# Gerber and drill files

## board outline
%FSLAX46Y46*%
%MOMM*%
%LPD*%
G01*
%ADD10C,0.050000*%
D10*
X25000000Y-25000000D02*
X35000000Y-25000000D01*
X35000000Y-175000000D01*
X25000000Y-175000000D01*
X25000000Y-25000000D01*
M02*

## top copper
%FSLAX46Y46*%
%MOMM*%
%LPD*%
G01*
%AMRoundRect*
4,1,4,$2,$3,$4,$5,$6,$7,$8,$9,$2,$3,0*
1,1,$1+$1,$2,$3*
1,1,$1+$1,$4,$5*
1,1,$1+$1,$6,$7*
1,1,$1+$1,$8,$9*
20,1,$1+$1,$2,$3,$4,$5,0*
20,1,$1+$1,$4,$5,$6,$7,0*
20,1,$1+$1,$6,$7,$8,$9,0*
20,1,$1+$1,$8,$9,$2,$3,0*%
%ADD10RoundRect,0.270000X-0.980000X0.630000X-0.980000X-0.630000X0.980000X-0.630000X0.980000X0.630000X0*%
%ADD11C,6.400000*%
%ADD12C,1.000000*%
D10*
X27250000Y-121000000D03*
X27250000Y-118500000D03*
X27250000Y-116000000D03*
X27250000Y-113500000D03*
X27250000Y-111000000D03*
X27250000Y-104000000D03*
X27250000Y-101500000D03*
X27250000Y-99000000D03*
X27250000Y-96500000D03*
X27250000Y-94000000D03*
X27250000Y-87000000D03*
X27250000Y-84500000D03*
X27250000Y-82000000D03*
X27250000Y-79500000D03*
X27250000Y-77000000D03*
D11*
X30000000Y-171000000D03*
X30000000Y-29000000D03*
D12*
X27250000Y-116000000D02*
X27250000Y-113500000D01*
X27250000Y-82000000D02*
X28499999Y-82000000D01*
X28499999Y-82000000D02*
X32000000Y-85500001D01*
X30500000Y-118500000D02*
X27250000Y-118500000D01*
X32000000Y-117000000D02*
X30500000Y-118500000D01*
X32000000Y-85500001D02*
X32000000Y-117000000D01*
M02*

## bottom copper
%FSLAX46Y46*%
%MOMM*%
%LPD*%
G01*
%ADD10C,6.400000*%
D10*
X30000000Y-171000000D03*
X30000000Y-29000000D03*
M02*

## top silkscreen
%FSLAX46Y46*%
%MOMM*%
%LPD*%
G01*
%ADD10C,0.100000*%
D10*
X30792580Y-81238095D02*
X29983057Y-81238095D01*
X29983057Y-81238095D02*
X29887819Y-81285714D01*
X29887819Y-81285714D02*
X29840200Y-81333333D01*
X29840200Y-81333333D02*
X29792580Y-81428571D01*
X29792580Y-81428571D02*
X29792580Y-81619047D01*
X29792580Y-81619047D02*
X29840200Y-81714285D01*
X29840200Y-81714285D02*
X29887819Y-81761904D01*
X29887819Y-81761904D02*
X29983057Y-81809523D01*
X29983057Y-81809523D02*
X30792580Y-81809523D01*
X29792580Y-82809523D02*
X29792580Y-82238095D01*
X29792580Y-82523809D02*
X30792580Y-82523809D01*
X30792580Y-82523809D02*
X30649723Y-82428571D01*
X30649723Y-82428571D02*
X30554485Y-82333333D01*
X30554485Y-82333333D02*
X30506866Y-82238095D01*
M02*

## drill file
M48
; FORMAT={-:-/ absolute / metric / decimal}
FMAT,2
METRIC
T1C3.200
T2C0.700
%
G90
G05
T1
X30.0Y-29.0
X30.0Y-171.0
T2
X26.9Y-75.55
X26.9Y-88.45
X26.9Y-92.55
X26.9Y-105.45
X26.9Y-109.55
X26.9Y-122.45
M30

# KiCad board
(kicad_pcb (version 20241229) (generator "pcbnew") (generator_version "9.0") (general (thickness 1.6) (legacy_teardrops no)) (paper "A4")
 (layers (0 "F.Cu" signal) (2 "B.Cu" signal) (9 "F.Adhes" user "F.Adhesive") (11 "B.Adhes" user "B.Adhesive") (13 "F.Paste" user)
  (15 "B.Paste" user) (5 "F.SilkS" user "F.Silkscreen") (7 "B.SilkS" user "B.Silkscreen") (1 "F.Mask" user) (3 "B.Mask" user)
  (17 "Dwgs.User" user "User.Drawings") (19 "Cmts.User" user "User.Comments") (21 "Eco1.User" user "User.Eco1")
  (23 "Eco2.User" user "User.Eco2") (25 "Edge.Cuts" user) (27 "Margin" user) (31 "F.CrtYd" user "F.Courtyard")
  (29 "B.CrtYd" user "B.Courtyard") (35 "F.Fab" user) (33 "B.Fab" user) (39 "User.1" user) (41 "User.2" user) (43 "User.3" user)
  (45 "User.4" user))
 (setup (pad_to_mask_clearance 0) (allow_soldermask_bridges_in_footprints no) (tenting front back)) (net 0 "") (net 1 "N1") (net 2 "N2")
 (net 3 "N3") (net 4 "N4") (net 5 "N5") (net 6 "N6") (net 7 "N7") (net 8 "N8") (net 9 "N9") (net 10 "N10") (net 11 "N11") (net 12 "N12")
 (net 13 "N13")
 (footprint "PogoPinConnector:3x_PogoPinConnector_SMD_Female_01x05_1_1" (layer "F.Cu") (at 27.25 77 -90)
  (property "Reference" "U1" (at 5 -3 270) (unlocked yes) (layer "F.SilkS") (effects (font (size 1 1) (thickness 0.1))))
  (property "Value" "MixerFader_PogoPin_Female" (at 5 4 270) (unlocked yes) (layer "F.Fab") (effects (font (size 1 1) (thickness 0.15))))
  (pad "" np_thru_hole circle (at -1.45 0.35 270) (size 0.7 0.7) (drill 0.7) (layers "*.Cu" "*.Mask"))
  (pad "" np_thru_hole circle (at 11.45 0.35 270) (size 0.7 0.7) (drill 0.7) (layers "*.Cu" "*.Mask"))
  (pad "" np_thru_hole circle (at 15.55 0.35 270) (size 0.7 0.7) (drill 0.7) (layers "*.Cu" "*.Mask"))
  (pad "" np_thru_hole circle (at 28.45 0.35 270) (size 0.7 0.7) (drill 0.7) (layers "*.Cu" "*.Mask"))
  (pad "" np_thru_hole circle (at 32.55 0.35 270) (size 0.7 0.7) (drill 0.7) (layers "*.Cu" "*.Mask"))
  (pad "" np_thru_hole circle (at 45.45 0.35 270) (size 0.7 0.7) (drill 0.7) (layers "*.Cu" "*.Mask"))
  (pad "1" smd roundrect (at 44 0 270) (size 1.8 2.5) (layers "F.Cu" "F.Mask" "F.Paste") (roundrect_rratio 0.15) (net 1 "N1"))
  (pad "2" smd roundrect (at 41.5 0 270) (size 1.8 2.5) (layers "F.Cu" "F.Mask" "F.Paste") (roundrect_rratio 0.15) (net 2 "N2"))
  (pad "3" smd roundrect (at 39 0 270) (size 1.8 2.5) (layers "F.Cu" "F.Mask" "F.Paste") (roundrect_rratio 0.15) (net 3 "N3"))
  (pad "4" smd roundrect (at 36.5 0 270) (size 1.8 2.5) (layers "F.Cu" "F.Mask" "F.Paste") (roundrect_rratio 0.15) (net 3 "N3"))
  (pad "5" smd roundrect (at 34 0 270) (size 1.8 2.5) (layers "F.Cu" "F.Mask" "F.Paste") (roundrect_rratio 0.15) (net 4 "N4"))
  (pad "6" smd roundrect (at 27 0 270) (size 1.8 2.5) (layers "F.Cu" "F.Mask" "F.Paste") (roundrect_rratio 0.15) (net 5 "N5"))
  (pad "7" smd roundrect (at 24.5 0 270) (size 1.8 2.5) (layers "F.Cu" "F.Mask" "F.Paste") (roundrect_rratio 0.15) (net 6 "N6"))
  (pad "8" smd roundrect (at 22 0 270) (size 1.8 2.5) (layers "F.Cu" "F.Mask" "F.Paste") (roundrect_rratio 0.15) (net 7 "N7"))
  (pad "9" smd roundrect (at 19.5 0 270) (size 1.8 2.5) (layers "F.Cu" "F.Mask" "F.Paste") (roundrect_rratio 0.15) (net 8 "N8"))
  (pad "10" smd roundrect (at 17 0 270) (size 1.8 2.5) (layers "F.Cu" "F.Mask" "F.Paste") (roundrect_rratio 0.15) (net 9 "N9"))
  (pad "11" smd roundrect (at 10 0 270) (size 1.8 2.5) (layers "F.Cu" "F.Mask" "F.Paste") (roundrect_rratio 0.15) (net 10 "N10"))
  (pad "12" smd roundrect (at 7.5 0 270) (size 1.8 2.5) (layers "F.Cu" "F.Mask" "F.Paste") (roundrect_rratio 0.15) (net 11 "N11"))
  (pad "13" smd roundrect (at 5 0 270) (size 1.8 2.5) (layers "F.Cu" "F.Mask" "F.Paste") (roundrect_rratio 0.15) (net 2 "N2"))
  (pad "14" smd roundrect (at 2.5 0 270) (size 1.8 2.5) (layers "F.Cu" "F.Mask" "F.Paste") (roundrect_rratio 0.15) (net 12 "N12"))
  (pad "15" smd roundrect (at 0 0 270) (size 1.8 2.5) (layers "F.Cu" "F.Mask" "F.Paste") (roundrect_rratio 0.15) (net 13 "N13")))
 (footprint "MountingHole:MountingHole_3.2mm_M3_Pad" (layer "F.Cu") (at 30 171)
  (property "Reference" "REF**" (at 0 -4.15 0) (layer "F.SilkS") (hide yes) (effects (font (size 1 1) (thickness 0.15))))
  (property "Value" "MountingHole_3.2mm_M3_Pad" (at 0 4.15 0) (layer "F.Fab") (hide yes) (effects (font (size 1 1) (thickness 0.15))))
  (pad "1" thru_hole circle (at 0 0) (size 6.4 6.4) (drill 3.2) (layers "*.Cu" "*.Mask") (remove_unused_layers no) (zone_connect 2)))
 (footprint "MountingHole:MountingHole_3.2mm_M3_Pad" (layer "F.Cu") (at 30 29)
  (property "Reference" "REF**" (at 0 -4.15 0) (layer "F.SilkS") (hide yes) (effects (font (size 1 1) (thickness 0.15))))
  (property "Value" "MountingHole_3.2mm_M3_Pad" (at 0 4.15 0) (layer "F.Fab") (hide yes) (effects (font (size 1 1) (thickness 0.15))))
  (pad "1" thru_hole circle (at 0 0) (size 6.4 6.4) (drill 3.2) (layers "*.Cu" "*.Mask") (remove_unused_layers no) (zone_connect 2)))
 (gr_rect (start 25 25) (end 35 175) (stroke (width 0.05) (type solid)) (fill no) (layer "Edge.Cuts"))
 (segment (start 27.25 116) (end 27.25 113.5) (width 1) (layer "F.Cu") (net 3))
 (segment (start 27.25 82) (end 28.499999 82) (width 1) (layer "F.Cu") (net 2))
 (segment (start 28.499999 82) (end 32 85.500001) (width 1) (layer "F.Cu") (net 2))
 (segment (start 30.5 118.5) (end 27.25 118.5) (width 1) (layer "F.Cu") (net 2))
 (segment (start 32 117) (end 30.5 118.5) (width 1) (layer "F.Cu") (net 2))
 (segment (start 32 85.500001) (end 32 117) (width 1) (layer "F.Cu") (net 2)))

